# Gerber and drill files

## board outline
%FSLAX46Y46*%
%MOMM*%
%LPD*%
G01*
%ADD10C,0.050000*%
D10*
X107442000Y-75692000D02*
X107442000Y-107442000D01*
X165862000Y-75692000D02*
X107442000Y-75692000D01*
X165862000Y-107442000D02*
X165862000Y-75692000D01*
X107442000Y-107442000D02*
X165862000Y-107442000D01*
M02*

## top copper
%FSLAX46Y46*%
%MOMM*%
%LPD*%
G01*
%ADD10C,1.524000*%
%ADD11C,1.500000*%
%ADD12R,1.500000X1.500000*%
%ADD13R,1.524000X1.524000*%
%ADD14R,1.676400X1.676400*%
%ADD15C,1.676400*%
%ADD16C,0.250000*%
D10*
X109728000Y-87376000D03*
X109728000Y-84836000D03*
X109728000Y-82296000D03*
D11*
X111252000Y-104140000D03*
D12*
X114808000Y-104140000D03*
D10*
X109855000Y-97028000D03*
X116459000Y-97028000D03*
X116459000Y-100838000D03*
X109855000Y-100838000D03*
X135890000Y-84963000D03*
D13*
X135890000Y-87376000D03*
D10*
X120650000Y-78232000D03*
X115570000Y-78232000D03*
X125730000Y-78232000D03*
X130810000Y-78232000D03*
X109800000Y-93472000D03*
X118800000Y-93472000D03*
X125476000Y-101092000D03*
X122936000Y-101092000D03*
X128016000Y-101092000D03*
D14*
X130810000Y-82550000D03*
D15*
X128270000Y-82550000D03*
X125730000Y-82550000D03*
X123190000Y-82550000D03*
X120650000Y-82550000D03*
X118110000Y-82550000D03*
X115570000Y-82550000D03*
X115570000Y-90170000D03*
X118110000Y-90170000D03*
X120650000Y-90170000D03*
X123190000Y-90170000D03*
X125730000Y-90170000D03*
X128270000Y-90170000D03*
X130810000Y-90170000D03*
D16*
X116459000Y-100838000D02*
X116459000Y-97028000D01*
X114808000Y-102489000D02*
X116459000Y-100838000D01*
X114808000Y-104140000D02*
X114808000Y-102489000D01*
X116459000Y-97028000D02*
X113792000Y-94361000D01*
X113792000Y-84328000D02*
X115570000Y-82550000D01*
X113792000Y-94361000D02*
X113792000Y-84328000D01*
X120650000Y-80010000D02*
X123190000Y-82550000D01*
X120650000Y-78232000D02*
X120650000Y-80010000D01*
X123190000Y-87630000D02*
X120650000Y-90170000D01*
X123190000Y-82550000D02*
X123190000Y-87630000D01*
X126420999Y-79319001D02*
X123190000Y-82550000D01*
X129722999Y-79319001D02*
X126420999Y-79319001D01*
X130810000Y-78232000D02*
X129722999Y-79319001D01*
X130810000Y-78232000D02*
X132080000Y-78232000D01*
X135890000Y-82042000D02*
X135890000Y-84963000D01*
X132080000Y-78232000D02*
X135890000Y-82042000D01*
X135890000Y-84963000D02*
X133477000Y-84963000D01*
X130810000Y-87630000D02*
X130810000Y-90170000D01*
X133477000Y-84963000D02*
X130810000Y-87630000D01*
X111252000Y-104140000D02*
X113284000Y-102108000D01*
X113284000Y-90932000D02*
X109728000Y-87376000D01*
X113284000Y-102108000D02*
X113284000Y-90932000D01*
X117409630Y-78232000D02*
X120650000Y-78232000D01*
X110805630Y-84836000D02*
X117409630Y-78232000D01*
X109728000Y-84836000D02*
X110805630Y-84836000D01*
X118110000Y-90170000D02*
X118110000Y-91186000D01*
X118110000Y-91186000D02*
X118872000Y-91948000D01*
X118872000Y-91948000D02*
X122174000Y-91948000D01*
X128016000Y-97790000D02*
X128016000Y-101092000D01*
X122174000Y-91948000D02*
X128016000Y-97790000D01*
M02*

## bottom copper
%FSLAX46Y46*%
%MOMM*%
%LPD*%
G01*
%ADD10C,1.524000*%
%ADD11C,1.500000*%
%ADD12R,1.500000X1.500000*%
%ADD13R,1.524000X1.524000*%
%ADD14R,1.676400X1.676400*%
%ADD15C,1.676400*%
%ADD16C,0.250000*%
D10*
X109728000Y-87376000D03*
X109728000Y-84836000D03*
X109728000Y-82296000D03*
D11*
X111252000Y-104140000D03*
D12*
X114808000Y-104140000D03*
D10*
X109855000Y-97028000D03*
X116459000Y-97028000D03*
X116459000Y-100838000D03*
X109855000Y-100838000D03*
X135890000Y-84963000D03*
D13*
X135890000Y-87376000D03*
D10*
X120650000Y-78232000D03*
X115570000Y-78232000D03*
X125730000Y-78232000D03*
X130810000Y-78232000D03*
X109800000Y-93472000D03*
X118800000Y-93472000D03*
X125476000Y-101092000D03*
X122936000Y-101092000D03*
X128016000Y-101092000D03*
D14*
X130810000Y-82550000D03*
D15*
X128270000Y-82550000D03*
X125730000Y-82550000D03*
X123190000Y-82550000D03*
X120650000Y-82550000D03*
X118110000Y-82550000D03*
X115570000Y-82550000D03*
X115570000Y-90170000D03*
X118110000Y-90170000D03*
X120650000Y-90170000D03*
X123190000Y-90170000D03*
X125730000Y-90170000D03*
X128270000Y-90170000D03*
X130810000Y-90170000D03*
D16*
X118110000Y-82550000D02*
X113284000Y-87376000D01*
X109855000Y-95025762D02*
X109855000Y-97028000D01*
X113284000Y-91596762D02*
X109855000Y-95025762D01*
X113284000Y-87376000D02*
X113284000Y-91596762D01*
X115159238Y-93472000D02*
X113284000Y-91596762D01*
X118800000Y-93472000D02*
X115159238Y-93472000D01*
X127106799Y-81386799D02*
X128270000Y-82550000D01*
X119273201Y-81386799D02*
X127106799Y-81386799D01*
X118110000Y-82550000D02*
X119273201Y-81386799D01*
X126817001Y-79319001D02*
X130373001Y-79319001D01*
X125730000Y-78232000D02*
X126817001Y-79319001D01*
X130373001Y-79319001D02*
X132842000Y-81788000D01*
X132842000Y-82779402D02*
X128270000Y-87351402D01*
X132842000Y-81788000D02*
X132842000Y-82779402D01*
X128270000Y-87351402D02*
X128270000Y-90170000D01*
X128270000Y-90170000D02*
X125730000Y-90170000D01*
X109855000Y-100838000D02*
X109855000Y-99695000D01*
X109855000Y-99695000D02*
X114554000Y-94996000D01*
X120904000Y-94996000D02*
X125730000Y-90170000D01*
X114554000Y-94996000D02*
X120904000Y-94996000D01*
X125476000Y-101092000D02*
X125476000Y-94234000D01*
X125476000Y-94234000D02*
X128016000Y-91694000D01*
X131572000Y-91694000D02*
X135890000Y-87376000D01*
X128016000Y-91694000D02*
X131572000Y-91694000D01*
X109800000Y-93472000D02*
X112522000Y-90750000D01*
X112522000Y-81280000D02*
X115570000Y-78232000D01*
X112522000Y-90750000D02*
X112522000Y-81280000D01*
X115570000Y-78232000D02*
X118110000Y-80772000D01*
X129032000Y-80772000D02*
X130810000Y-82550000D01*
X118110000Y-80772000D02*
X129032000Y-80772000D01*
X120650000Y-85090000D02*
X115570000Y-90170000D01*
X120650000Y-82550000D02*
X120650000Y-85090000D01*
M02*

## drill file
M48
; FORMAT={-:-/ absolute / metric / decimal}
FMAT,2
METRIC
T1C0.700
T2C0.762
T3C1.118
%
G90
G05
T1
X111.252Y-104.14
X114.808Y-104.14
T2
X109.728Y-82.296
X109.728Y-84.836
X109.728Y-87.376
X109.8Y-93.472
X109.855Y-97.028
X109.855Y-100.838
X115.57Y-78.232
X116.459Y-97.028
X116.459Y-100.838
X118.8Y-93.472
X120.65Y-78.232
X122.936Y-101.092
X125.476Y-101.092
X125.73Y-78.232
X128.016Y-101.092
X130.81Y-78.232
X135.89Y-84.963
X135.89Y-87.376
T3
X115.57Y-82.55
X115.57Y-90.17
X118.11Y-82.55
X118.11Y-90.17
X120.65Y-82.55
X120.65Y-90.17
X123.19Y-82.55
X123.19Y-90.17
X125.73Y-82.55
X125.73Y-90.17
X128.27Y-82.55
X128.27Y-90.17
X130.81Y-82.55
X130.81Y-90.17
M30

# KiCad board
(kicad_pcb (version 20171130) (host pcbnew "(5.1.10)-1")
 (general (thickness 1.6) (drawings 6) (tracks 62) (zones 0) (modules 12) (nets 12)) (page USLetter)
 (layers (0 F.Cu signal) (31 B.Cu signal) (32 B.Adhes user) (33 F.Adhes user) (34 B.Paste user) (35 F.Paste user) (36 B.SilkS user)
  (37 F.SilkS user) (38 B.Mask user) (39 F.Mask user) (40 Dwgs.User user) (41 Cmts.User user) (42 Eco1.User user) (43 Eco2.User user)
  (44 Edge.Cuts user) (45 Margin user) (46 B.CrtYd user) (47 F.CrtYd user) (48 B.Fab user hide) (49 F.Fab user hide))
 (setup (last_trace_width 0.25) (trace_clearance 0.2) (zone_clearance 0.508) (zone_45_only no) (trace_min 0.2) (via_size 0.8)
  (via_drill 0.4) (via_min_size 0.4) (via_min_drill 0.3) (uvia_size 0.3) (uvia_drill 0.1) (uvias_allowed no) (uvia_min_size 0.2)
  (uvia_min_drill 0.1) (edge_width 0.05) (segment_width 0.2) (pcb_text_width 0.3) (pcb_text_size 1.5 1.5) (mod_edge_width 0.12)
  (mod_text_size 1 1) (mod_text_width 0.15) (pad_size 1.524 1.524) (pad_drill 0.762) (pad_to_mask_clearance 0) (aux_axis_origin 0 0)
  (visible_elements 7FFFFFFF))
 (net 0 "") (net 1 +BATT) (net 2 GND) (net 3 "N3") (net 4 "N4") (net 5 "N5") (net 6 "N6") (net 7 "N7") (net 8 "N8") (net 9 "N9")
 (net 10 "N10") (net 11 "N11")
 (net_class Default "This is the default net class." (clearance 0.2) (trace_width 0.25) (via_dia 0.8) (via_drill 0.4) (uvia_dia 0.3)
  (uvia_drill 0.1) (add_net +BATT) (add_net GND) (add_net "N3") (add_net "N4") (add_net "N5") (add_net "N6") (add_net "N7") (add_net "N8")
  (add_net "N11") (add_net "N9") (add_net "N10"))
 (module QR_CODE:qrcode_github (layer F.Cu) (at 154.178 86.614)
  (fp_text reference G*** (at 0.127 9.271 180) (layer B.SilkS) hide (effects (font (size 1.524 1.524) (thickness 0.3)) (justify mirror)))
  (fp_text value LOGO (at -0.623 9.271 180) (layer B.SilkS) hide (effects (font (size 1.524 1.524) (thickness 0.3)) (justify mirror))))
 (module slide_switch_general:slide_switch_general (layer F.Cu) (at 109.728 84.836 270)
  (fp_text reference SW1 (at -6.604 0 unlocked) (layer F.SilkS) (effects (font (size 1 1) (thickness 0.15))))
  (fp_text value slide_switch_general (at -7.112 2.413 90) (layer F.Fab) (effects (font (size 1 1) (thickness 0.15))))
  (pad 3 thru_hole circle (at 2.54 0 270) (size 1.524 1.524) (drill 0.762) (layers *.Cu *.Mask) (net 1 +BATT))
  (pad 2 thru_hole circle (at 0 0 270) (size 1.524 1.524) (drill 0.762) (layers *.Cu *.Mask) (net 1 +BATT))
  (pad 1 thru_hole circle (at -2.54 0 270) (size 1.524 1.524) (drill 0.762) (layers *.Cu *.Mask)))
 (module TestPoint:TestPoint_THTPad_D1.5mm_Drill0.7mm (layer F.Cu) (at 111.252 104.14)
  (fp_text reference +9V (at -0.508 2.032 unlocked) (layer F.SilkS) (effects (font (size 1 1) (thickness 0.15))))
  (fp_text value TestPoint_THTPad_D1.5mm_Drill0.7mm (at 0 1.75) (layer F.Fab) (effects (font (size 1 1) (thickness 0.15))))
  (pad 1 thru_hole circle (at 0 0) (size 1.5 1.5) (drill 0.7) (layers *.Cu *.Mask) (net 1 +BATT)))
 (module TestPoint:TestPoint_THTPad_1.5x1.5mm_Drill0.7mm (layer F.Cu) (at 114.808 104.14)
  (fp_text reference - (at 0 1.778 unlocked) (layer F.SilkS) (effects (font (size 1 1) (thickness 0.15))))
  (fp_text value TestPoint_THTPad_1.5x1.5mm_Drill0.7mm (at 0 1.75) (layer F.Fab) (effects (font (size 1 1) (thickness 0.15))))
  (pad 1 thru_hole rect (at 0 0) (size 1.5 1.5) (drill 0.7) (layers *.Cu *.Mask) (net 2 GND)))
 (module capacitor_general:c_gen (layer F.Cu) (at 113.284 97.028)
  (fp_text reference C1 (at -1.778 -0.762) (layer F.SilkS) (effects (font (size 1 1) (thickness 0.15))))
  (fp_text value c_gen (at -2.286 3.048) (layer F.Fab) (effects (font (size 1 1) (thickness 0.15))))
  (pad 1 thru_hole circle (at -3.429 0) (size 1.524 1.524) (drill 0.762) (layers *.Cu *.Mask) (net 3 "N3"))
  (pad 2 thru_hole circle (at 3.175 0) (size 1.524 1.524) (drill 0.762) (layers *.Cu *.Mask) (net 2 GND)))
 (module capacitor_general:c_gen (layer F.Cu) (at 113.284 100.838)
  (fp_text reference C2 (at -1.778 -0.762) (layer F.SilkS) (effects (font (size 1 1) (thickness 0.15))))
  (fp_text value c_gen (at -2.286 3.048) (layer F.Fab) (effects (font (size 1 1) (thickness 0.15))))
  (pad 2 thru_hole circle (at 3.175 0) (size 1.524 1.524) (drill 0.762) (layers *.Cu *.Mask) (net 2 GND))
  (pad 1 thru_hole circle (at -3.429 0) (size 1.524 1.524) (drill 0.762) (layers *.Cu *.Mask) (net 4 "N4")))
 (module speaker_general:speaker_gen (layer F.Cu) (at 135.89 86.106 270)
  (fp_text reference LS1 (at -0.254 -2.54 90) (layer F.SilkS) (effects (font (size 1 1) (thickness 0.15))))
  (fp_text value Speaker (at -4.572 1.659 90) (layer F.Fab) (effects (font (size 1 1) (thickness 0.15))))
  (pad 1 thru_hole circle (at -1.143 0 270) (size 1.524 1.524) (drill 0.762) (layers *.Cu *.Mask) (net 1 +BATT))
  (pad 2 thru_hole rect (at 1.27 0 270) (size 1.524 1.524) (drill 0.762) (layers *.Cu *.Mask) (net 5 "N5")))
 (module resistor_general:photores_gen (layer F.Cu) (at 118.11 78.232 180)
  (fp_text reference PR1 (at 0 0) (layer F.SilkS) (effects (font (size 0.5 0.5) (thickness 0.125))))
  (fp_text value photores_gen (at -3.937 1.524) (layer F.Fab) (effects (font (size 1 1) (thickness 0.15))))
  (pad 1 thru_hole circle (at -2.54 0 180) (size 1.524 1.524) (drill 0.762) (layers *.Cu *.Mask) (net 1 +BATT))
  (pad 2 thru_hole circle (at 2.54 0 180) (size 1.524 1.524) (drill 0.762) (layers *.Cu *.Mask) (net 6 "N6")))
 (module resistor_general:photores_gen (layer F.Cu) (at 128.27 78.232 180)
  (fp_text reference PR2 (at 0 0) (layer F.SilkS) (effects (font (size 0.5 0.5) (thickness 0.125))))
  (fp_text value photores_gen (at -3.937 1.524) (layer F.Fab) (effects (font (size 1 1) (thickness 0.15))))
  (pad 2 thru_hole circle (at 2.54 0 180) (size 1.524 1.524) (drill 0.762) (layers *.Cu *.Mask) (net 4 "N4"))
  (pad 1 thru_hole circle (at -2.54 0 180) (size 1.524 1.524) (drill 0.762) (layers *.Cu *.Mask) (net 1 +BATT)))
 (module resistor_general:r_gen (layer F.Cu) (at 114.3 93.472)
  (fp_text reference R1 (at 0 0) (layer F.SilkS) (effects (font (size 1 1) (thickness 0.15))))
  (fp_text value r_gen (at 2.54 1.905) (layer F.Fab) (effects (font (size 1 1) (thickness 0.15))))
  (pad 1 thru_hole circle (at -4.5 0) (size 1.524 1.524) (drill 0.762) (layers *.Cu *.Mask) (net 6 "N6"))
  (pad 2 thru_hole circle (at 4.5 0) (size 1.524 1.524) (drill 0.762) (layers *.Cu *.Mask) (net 3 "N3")))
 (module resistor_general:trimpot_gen (layer F.Cu) (at 125.476 102.108)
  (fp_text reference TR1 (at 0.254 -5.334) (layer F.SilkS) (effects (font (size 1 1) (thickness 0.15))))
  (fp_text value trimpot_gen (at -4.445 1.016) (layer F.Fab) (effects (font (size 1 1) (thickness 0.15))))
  (pad 2 thru_hole circle (at 0 -1.016) (size 1.524 1.524) (drill 0.762) (layers *.Cu *.Mask) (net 5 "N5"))
  (pad 1 thru_hole circle (at -2.54 -1.016) (size 1.524 1.524) (drill 0.762) (layers *.Cu *.Mask) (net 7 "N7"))
  (pad 3 thru_hole circle (at 2.54 -1.016) (size 1.524 1.524) (drill 0.762) (layers *.Cu *.Mask) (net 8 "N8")))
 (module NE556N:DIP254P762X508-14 (layer F.Cu) (at 115.57 90.17 270)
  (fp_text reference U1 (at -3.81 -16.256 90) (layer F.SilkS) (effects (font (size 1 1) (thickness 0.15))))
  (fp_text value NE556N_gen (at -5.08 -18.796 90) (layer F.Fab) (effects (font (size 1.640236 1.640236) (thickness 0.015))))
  (pad 1 thru_hole rect (at -7.62 -15.24 270) (size 1.6764 1.6764) (drill 1.1176) (layers *.Cu *.Mask) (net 6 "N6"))
  (pad 2 thru_hole circle (at -7.62 -12.7 270) (size 1.6764 1.6764) (drill 1.1176) (layers *.Cu *.Mask) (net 3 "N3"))
  (pad 3 thru_hole circle (at -7.62 -10.16 270) (size 1.6764 1.6764) (drill 1.1176) (layers *.Cu *.Mask) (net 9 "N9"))
  (pad 4 thru_hole circle (at -7.62 -7.62 270) (size 1.6764 1.6764) (drill 1.1176) (layers *.Cu *.Mask) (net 1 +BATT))
  (pad 5 thru_hole circle (at -7.62 -5.08 270) (size 1.6764 1.6764) (drill 1.1176) (layers *.Cu *.Mask) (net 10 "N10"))
  (pad 6 thru_hole circle (at -7.62 -2.54 270) (size 1.6764 1.6764) (drill 1.1176) (layers *.Cu *.Mask) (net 3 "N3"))
  (pad 7 thru_hole circle (at -7.62 0 270) (size 1.6764 1.6764) (drill 1.1176) (layers *.Cu *.Mask) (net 2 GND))
  (pad 8 thru_hole circle (at 0 0 270) (size 1.6764 1.6764) (drill 1.1176) (layers *.Cu *.Mask) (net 10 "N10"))
  (pad 9 thru_hole circle (at 0 -2.54 270) (size 1.6764 1.6764) (drill 1.1176) (layers *.Cu *.Mask) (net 8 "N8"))
  (pad 10 thru_hole circle (at 0 -5.08 270) (size 1.6764 1.6764) (drill 1.1176) (layers *.Cu *.Mask) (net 1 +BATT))
  (pad 11 thru_hole circle (at 0 -7.62 270) (size 1.6764 1.6764) (drill 1.1176) (layers *.Cu *.Mask) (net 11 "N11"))
  (pad 12 thru_hole circle (at 0 -10.16 270) (size 1.6764 1.6764) (drill 1.1176) (layers *.Cu *.Mask) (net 4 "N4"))
  (pad 13 thru_hole circle (at 0 -12.7 270) (size 1.6764 1.6764) (drill 1.1176) (layers *.Cu *.Mask) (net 4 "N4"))
  (pad 14 thru_hole circle (at 0 -15.24 270) (size 1.6764 1.6764) (drill 1.1176) (layers *.Cu *.Mask) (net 1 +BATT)))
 (gr_line (start 107.442 75.692) (end 107.442 107.442) (layer Edge.Cuts) (width 0.05))
 (gr_line (start 165.862 75.692) (end 107.442 75.692) (layer Edge.Cuts) (width 0.05))
 (gr_line (start 165.862 107.442) (end 165.862 75.692) (layer Edge.Cuts) (width 0.05))
 (gr_line (start 107.442 107.442) (end 165.862 107.442) (layer Edge.Cuts) (width 0.05))
 (segment (start 118.11 82.55) (end 113.284 87.376) (width 0.25) (layer B.Cu) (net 3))
 (segment (start 109.855 95.025762) (end 109.855 97.028) (width 0.25) (layer B.Cu) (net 3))
 (segment (start 113.284 91.596762) (end 109.855 95.025762) (width 0.25) (layer B.Cu) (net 3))
 (segment (start 113.284 87.376) (end 113.284 91.596762) (width 0.25) (layer B.Cu) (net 3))
 (segment (start 115.159238 93.472) (end 113.284 91.596762) (width 0.25) (layer B.Cu) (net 3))
 (segment (start 118.8 93.472) (end 115.159238 93.472) (width 0.25) (layer B.Cu) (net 3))
 (segment (start 127.106799 81.386799) (end 128.27 82.55) (width 0.25) (layer B.Cu) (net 3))
 (segment (start 119.273201 81.386799) (end 127.106799 81.386799) (width 0.25) (layer B.Cu) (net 3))
 (segment (start 118.11 82.55) (end 119.273201 81.386799) (width 0.25) (layer B.Cu) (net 3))
 (segment (start 116.459 100.838) (end 116.459 97.028) (width 0.25) (layer F.Cu) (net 2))
 (segment (start 114.808 102.489) (end 116.459 100.838) (width 0.25) (layer F.Cu) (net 2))
 (segment (start 114.808 104.14) (end 114.808 102.489) (width 0.25) (layer F.Cu) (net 2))
 (segment (start 116.459 97.028) (end 113.792 94.361) (width 0.25) (layer F.Cu) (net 2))
 (segment (start 113.792 84.328) (end 115.57 82.55) (width 0.25) (layer F.Cu) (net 2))
 (segment (start 113.792 94.361) (end 113.792 84.328) (width 0.25) (layer F.Cu) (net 2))
 (segment (start 126.817001 79.319001) (end 130.373001 79.319001) (width 0.25) (layer B.Cu) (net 4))
 (segment (start 125.73 78.232) (end 126.817001 79.319001) (width 0.25) (layer B.Cu) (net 4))
 (segment (start 130.373001 79.319001) (end 132.842 81.788) (width 0.25) (layer B.Cu) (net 4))
 (segment (start 132.842 82.779402) (end 128.27 87.351402) (width 0.25) (layer B.Cu) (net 4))
 (segment (start 132.842 81.788) (end 132.842 82.779402) (width 0.25) (layer B.Cu) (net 4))
 (segment (start 128.27 87.351402) (end 128.27 90.17) (width 0.25) (layer B.Cu) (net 4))
 (segment (start 128.27 90.17) (end 125.73 90.17) (width 0.25) (layer B.Cu) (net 4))
 (segment (start 109.855 100.838) (end 109.855 99.695) (width 0.25) (layer B.Cu) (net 4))
 (segment (start 109.855 99.695) (end 114.554 94.996) (width 0.25) (layer B.Cu) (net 4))
 (segment (start 120.904 94.996) (end 125.73 90.17) (width 0.25) (layer B.Cu) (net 4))
 (segment (start 114.554 94.996) (end 120.904 94.996) (width 0.25) (layer B.Cu) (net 4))
 (segment (start 120.65 80.01) (end 123.19 82.55) (width 0.25) (layer F.Cu) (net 1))
 (segment (start 120.65 78.232) (end 120.65 80.01) (width 0.25) (layer F.Cu) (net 1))
 (segment (start 123.19 87.63) (end 120.65 90.17) (width 0.25) (layer F.Cu) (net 1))
 (segment (start 123.19 82.55) (end 123.19 87.63) (width 0.25) (layer F.Cu) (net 1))
 (segment (start 126.420999 79.319001) (end 123.19 82.55) (width 0.25) (layer F.Cu) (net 1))
 (segment (start 129.722999 79.319001) (end 126.420999 79.319001) (width 0.25) (layer F.Cu) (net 1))
 (segment (start 130.81 78.232) (end 129.722999 79.319001) (width 0.25) (layer F.Cu) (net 1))
 (segment (start 130.81 78.232) (end 132.08 78.232) (width 0.25) (layer F.Cu) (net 1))
 (segment (start 135.89 82.042) (end 135.89 84.963) (width 0.25) (layer F.Cu) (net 1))
 (segment (start 132.08 78.232) (end 135.89 82.042) (width 0.25) (layer F.Cu) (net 1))
 (segment (start 135.89 84.963) (end 133.477 84.963) (width 0.25) (layer F.Cu) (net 1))
 (segment (start 130.81 87.63) (end 130.81 90.17) (width 0.25) (layer F.Cu) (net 1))
 (segment (start 133.477 84.963) (end 130.81 87.63) (width 0.25) (layer F.Cu) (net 1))
 (segment (start 111.252 104.14) (end 113.284 102.108) (width 0.25) (layer F.Cu) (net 1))
 (segment (start 113.284 90.932) (end 109.728 87.376) (width 0.25) (layer F.Cu) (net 1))
 (segment (start 113.284 102.108) (end 113.284 90.932) (width 0.25) (layer F.Cu) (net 1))
 (segment (start 117.40963 78.232) (end 120.65 78.232) (width 0.25) (layer F.Cu) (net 1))
 (segment (start 110.80563 84.836) (end 117.40963 78.232) (width 0.25) (layer F.Cu) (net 1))
 (segment (start 109.728 84.836) (end 110.80563 84.836) (width 0.25) (layer F.Cu) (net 1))
 (segment (start 125.476 101.092) (end 125.476 94.234) (width 0.25) (layer B.Cu) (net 5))
 (segment (start 125.476 94.234) (end 128.016 91.694) (width 0.25) (layer B.Cu) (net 5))
 (segment (start 131.572 91.694) (end 135.89 87.376) (width 0.25) (layer B.Cu) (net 5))
 (segment (start 128.016 91.694) (end 131.572 91.694) (width 0.25) (layer B.Cu) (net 5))
 (segment (start 109.8 93.472) (end 112.522 90.75) (width 0.25) (layer B.Cu) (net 6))
 (segment (start 112.522 81.28) (end 115.57 78.232) (width 0.25) (layer B.Cu) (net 6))
 (segment (start 112.522 90.75) (end 112.522 81.28) (width 0.25) (layer B.Cu) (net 6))
 (segment (start 115.57 78.232) (end 118.11 80.772) (width 0.25) (layer B.Cu) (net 6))
 (segment (start 129.032 80.772) (end 130.81 82.55) (width 0.25) (layer B.Cu) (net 6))
 (segment (start 118.11 80.772) (end 129.032 80.772) (width 0.25) (layer B.Cu) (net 6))
 (segment (start 118.11 90.17) (end 118.11 91.186) (width 0.25) (layer F.Cu) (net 8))
 (segment (start 118.11 91.186) (end 118.872 91.948) (width 0.25) (layer F.Cu) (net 8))
 (segment (start 118.872 91.948) (end 122.174 91.948) (width 0.25) (layer F.Cu) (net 8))
 (segment (start 128.016 97.79) (end 128.016 101.092) (width 0.25) (layer F.Cu) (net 8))
 (segment (start 122.174 91.948) (end 128.016 97.79) (width 0.25) (layer F.Cu) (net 8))
 (segment (start 120.65 85.09) (end 115.57 90.17) (width 0.25) (layer B.Cu) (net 10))
 (segment (start 120.65 82.55) (end 120.65 85.09) (width 0.25) (layer B.Cu) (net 10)))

